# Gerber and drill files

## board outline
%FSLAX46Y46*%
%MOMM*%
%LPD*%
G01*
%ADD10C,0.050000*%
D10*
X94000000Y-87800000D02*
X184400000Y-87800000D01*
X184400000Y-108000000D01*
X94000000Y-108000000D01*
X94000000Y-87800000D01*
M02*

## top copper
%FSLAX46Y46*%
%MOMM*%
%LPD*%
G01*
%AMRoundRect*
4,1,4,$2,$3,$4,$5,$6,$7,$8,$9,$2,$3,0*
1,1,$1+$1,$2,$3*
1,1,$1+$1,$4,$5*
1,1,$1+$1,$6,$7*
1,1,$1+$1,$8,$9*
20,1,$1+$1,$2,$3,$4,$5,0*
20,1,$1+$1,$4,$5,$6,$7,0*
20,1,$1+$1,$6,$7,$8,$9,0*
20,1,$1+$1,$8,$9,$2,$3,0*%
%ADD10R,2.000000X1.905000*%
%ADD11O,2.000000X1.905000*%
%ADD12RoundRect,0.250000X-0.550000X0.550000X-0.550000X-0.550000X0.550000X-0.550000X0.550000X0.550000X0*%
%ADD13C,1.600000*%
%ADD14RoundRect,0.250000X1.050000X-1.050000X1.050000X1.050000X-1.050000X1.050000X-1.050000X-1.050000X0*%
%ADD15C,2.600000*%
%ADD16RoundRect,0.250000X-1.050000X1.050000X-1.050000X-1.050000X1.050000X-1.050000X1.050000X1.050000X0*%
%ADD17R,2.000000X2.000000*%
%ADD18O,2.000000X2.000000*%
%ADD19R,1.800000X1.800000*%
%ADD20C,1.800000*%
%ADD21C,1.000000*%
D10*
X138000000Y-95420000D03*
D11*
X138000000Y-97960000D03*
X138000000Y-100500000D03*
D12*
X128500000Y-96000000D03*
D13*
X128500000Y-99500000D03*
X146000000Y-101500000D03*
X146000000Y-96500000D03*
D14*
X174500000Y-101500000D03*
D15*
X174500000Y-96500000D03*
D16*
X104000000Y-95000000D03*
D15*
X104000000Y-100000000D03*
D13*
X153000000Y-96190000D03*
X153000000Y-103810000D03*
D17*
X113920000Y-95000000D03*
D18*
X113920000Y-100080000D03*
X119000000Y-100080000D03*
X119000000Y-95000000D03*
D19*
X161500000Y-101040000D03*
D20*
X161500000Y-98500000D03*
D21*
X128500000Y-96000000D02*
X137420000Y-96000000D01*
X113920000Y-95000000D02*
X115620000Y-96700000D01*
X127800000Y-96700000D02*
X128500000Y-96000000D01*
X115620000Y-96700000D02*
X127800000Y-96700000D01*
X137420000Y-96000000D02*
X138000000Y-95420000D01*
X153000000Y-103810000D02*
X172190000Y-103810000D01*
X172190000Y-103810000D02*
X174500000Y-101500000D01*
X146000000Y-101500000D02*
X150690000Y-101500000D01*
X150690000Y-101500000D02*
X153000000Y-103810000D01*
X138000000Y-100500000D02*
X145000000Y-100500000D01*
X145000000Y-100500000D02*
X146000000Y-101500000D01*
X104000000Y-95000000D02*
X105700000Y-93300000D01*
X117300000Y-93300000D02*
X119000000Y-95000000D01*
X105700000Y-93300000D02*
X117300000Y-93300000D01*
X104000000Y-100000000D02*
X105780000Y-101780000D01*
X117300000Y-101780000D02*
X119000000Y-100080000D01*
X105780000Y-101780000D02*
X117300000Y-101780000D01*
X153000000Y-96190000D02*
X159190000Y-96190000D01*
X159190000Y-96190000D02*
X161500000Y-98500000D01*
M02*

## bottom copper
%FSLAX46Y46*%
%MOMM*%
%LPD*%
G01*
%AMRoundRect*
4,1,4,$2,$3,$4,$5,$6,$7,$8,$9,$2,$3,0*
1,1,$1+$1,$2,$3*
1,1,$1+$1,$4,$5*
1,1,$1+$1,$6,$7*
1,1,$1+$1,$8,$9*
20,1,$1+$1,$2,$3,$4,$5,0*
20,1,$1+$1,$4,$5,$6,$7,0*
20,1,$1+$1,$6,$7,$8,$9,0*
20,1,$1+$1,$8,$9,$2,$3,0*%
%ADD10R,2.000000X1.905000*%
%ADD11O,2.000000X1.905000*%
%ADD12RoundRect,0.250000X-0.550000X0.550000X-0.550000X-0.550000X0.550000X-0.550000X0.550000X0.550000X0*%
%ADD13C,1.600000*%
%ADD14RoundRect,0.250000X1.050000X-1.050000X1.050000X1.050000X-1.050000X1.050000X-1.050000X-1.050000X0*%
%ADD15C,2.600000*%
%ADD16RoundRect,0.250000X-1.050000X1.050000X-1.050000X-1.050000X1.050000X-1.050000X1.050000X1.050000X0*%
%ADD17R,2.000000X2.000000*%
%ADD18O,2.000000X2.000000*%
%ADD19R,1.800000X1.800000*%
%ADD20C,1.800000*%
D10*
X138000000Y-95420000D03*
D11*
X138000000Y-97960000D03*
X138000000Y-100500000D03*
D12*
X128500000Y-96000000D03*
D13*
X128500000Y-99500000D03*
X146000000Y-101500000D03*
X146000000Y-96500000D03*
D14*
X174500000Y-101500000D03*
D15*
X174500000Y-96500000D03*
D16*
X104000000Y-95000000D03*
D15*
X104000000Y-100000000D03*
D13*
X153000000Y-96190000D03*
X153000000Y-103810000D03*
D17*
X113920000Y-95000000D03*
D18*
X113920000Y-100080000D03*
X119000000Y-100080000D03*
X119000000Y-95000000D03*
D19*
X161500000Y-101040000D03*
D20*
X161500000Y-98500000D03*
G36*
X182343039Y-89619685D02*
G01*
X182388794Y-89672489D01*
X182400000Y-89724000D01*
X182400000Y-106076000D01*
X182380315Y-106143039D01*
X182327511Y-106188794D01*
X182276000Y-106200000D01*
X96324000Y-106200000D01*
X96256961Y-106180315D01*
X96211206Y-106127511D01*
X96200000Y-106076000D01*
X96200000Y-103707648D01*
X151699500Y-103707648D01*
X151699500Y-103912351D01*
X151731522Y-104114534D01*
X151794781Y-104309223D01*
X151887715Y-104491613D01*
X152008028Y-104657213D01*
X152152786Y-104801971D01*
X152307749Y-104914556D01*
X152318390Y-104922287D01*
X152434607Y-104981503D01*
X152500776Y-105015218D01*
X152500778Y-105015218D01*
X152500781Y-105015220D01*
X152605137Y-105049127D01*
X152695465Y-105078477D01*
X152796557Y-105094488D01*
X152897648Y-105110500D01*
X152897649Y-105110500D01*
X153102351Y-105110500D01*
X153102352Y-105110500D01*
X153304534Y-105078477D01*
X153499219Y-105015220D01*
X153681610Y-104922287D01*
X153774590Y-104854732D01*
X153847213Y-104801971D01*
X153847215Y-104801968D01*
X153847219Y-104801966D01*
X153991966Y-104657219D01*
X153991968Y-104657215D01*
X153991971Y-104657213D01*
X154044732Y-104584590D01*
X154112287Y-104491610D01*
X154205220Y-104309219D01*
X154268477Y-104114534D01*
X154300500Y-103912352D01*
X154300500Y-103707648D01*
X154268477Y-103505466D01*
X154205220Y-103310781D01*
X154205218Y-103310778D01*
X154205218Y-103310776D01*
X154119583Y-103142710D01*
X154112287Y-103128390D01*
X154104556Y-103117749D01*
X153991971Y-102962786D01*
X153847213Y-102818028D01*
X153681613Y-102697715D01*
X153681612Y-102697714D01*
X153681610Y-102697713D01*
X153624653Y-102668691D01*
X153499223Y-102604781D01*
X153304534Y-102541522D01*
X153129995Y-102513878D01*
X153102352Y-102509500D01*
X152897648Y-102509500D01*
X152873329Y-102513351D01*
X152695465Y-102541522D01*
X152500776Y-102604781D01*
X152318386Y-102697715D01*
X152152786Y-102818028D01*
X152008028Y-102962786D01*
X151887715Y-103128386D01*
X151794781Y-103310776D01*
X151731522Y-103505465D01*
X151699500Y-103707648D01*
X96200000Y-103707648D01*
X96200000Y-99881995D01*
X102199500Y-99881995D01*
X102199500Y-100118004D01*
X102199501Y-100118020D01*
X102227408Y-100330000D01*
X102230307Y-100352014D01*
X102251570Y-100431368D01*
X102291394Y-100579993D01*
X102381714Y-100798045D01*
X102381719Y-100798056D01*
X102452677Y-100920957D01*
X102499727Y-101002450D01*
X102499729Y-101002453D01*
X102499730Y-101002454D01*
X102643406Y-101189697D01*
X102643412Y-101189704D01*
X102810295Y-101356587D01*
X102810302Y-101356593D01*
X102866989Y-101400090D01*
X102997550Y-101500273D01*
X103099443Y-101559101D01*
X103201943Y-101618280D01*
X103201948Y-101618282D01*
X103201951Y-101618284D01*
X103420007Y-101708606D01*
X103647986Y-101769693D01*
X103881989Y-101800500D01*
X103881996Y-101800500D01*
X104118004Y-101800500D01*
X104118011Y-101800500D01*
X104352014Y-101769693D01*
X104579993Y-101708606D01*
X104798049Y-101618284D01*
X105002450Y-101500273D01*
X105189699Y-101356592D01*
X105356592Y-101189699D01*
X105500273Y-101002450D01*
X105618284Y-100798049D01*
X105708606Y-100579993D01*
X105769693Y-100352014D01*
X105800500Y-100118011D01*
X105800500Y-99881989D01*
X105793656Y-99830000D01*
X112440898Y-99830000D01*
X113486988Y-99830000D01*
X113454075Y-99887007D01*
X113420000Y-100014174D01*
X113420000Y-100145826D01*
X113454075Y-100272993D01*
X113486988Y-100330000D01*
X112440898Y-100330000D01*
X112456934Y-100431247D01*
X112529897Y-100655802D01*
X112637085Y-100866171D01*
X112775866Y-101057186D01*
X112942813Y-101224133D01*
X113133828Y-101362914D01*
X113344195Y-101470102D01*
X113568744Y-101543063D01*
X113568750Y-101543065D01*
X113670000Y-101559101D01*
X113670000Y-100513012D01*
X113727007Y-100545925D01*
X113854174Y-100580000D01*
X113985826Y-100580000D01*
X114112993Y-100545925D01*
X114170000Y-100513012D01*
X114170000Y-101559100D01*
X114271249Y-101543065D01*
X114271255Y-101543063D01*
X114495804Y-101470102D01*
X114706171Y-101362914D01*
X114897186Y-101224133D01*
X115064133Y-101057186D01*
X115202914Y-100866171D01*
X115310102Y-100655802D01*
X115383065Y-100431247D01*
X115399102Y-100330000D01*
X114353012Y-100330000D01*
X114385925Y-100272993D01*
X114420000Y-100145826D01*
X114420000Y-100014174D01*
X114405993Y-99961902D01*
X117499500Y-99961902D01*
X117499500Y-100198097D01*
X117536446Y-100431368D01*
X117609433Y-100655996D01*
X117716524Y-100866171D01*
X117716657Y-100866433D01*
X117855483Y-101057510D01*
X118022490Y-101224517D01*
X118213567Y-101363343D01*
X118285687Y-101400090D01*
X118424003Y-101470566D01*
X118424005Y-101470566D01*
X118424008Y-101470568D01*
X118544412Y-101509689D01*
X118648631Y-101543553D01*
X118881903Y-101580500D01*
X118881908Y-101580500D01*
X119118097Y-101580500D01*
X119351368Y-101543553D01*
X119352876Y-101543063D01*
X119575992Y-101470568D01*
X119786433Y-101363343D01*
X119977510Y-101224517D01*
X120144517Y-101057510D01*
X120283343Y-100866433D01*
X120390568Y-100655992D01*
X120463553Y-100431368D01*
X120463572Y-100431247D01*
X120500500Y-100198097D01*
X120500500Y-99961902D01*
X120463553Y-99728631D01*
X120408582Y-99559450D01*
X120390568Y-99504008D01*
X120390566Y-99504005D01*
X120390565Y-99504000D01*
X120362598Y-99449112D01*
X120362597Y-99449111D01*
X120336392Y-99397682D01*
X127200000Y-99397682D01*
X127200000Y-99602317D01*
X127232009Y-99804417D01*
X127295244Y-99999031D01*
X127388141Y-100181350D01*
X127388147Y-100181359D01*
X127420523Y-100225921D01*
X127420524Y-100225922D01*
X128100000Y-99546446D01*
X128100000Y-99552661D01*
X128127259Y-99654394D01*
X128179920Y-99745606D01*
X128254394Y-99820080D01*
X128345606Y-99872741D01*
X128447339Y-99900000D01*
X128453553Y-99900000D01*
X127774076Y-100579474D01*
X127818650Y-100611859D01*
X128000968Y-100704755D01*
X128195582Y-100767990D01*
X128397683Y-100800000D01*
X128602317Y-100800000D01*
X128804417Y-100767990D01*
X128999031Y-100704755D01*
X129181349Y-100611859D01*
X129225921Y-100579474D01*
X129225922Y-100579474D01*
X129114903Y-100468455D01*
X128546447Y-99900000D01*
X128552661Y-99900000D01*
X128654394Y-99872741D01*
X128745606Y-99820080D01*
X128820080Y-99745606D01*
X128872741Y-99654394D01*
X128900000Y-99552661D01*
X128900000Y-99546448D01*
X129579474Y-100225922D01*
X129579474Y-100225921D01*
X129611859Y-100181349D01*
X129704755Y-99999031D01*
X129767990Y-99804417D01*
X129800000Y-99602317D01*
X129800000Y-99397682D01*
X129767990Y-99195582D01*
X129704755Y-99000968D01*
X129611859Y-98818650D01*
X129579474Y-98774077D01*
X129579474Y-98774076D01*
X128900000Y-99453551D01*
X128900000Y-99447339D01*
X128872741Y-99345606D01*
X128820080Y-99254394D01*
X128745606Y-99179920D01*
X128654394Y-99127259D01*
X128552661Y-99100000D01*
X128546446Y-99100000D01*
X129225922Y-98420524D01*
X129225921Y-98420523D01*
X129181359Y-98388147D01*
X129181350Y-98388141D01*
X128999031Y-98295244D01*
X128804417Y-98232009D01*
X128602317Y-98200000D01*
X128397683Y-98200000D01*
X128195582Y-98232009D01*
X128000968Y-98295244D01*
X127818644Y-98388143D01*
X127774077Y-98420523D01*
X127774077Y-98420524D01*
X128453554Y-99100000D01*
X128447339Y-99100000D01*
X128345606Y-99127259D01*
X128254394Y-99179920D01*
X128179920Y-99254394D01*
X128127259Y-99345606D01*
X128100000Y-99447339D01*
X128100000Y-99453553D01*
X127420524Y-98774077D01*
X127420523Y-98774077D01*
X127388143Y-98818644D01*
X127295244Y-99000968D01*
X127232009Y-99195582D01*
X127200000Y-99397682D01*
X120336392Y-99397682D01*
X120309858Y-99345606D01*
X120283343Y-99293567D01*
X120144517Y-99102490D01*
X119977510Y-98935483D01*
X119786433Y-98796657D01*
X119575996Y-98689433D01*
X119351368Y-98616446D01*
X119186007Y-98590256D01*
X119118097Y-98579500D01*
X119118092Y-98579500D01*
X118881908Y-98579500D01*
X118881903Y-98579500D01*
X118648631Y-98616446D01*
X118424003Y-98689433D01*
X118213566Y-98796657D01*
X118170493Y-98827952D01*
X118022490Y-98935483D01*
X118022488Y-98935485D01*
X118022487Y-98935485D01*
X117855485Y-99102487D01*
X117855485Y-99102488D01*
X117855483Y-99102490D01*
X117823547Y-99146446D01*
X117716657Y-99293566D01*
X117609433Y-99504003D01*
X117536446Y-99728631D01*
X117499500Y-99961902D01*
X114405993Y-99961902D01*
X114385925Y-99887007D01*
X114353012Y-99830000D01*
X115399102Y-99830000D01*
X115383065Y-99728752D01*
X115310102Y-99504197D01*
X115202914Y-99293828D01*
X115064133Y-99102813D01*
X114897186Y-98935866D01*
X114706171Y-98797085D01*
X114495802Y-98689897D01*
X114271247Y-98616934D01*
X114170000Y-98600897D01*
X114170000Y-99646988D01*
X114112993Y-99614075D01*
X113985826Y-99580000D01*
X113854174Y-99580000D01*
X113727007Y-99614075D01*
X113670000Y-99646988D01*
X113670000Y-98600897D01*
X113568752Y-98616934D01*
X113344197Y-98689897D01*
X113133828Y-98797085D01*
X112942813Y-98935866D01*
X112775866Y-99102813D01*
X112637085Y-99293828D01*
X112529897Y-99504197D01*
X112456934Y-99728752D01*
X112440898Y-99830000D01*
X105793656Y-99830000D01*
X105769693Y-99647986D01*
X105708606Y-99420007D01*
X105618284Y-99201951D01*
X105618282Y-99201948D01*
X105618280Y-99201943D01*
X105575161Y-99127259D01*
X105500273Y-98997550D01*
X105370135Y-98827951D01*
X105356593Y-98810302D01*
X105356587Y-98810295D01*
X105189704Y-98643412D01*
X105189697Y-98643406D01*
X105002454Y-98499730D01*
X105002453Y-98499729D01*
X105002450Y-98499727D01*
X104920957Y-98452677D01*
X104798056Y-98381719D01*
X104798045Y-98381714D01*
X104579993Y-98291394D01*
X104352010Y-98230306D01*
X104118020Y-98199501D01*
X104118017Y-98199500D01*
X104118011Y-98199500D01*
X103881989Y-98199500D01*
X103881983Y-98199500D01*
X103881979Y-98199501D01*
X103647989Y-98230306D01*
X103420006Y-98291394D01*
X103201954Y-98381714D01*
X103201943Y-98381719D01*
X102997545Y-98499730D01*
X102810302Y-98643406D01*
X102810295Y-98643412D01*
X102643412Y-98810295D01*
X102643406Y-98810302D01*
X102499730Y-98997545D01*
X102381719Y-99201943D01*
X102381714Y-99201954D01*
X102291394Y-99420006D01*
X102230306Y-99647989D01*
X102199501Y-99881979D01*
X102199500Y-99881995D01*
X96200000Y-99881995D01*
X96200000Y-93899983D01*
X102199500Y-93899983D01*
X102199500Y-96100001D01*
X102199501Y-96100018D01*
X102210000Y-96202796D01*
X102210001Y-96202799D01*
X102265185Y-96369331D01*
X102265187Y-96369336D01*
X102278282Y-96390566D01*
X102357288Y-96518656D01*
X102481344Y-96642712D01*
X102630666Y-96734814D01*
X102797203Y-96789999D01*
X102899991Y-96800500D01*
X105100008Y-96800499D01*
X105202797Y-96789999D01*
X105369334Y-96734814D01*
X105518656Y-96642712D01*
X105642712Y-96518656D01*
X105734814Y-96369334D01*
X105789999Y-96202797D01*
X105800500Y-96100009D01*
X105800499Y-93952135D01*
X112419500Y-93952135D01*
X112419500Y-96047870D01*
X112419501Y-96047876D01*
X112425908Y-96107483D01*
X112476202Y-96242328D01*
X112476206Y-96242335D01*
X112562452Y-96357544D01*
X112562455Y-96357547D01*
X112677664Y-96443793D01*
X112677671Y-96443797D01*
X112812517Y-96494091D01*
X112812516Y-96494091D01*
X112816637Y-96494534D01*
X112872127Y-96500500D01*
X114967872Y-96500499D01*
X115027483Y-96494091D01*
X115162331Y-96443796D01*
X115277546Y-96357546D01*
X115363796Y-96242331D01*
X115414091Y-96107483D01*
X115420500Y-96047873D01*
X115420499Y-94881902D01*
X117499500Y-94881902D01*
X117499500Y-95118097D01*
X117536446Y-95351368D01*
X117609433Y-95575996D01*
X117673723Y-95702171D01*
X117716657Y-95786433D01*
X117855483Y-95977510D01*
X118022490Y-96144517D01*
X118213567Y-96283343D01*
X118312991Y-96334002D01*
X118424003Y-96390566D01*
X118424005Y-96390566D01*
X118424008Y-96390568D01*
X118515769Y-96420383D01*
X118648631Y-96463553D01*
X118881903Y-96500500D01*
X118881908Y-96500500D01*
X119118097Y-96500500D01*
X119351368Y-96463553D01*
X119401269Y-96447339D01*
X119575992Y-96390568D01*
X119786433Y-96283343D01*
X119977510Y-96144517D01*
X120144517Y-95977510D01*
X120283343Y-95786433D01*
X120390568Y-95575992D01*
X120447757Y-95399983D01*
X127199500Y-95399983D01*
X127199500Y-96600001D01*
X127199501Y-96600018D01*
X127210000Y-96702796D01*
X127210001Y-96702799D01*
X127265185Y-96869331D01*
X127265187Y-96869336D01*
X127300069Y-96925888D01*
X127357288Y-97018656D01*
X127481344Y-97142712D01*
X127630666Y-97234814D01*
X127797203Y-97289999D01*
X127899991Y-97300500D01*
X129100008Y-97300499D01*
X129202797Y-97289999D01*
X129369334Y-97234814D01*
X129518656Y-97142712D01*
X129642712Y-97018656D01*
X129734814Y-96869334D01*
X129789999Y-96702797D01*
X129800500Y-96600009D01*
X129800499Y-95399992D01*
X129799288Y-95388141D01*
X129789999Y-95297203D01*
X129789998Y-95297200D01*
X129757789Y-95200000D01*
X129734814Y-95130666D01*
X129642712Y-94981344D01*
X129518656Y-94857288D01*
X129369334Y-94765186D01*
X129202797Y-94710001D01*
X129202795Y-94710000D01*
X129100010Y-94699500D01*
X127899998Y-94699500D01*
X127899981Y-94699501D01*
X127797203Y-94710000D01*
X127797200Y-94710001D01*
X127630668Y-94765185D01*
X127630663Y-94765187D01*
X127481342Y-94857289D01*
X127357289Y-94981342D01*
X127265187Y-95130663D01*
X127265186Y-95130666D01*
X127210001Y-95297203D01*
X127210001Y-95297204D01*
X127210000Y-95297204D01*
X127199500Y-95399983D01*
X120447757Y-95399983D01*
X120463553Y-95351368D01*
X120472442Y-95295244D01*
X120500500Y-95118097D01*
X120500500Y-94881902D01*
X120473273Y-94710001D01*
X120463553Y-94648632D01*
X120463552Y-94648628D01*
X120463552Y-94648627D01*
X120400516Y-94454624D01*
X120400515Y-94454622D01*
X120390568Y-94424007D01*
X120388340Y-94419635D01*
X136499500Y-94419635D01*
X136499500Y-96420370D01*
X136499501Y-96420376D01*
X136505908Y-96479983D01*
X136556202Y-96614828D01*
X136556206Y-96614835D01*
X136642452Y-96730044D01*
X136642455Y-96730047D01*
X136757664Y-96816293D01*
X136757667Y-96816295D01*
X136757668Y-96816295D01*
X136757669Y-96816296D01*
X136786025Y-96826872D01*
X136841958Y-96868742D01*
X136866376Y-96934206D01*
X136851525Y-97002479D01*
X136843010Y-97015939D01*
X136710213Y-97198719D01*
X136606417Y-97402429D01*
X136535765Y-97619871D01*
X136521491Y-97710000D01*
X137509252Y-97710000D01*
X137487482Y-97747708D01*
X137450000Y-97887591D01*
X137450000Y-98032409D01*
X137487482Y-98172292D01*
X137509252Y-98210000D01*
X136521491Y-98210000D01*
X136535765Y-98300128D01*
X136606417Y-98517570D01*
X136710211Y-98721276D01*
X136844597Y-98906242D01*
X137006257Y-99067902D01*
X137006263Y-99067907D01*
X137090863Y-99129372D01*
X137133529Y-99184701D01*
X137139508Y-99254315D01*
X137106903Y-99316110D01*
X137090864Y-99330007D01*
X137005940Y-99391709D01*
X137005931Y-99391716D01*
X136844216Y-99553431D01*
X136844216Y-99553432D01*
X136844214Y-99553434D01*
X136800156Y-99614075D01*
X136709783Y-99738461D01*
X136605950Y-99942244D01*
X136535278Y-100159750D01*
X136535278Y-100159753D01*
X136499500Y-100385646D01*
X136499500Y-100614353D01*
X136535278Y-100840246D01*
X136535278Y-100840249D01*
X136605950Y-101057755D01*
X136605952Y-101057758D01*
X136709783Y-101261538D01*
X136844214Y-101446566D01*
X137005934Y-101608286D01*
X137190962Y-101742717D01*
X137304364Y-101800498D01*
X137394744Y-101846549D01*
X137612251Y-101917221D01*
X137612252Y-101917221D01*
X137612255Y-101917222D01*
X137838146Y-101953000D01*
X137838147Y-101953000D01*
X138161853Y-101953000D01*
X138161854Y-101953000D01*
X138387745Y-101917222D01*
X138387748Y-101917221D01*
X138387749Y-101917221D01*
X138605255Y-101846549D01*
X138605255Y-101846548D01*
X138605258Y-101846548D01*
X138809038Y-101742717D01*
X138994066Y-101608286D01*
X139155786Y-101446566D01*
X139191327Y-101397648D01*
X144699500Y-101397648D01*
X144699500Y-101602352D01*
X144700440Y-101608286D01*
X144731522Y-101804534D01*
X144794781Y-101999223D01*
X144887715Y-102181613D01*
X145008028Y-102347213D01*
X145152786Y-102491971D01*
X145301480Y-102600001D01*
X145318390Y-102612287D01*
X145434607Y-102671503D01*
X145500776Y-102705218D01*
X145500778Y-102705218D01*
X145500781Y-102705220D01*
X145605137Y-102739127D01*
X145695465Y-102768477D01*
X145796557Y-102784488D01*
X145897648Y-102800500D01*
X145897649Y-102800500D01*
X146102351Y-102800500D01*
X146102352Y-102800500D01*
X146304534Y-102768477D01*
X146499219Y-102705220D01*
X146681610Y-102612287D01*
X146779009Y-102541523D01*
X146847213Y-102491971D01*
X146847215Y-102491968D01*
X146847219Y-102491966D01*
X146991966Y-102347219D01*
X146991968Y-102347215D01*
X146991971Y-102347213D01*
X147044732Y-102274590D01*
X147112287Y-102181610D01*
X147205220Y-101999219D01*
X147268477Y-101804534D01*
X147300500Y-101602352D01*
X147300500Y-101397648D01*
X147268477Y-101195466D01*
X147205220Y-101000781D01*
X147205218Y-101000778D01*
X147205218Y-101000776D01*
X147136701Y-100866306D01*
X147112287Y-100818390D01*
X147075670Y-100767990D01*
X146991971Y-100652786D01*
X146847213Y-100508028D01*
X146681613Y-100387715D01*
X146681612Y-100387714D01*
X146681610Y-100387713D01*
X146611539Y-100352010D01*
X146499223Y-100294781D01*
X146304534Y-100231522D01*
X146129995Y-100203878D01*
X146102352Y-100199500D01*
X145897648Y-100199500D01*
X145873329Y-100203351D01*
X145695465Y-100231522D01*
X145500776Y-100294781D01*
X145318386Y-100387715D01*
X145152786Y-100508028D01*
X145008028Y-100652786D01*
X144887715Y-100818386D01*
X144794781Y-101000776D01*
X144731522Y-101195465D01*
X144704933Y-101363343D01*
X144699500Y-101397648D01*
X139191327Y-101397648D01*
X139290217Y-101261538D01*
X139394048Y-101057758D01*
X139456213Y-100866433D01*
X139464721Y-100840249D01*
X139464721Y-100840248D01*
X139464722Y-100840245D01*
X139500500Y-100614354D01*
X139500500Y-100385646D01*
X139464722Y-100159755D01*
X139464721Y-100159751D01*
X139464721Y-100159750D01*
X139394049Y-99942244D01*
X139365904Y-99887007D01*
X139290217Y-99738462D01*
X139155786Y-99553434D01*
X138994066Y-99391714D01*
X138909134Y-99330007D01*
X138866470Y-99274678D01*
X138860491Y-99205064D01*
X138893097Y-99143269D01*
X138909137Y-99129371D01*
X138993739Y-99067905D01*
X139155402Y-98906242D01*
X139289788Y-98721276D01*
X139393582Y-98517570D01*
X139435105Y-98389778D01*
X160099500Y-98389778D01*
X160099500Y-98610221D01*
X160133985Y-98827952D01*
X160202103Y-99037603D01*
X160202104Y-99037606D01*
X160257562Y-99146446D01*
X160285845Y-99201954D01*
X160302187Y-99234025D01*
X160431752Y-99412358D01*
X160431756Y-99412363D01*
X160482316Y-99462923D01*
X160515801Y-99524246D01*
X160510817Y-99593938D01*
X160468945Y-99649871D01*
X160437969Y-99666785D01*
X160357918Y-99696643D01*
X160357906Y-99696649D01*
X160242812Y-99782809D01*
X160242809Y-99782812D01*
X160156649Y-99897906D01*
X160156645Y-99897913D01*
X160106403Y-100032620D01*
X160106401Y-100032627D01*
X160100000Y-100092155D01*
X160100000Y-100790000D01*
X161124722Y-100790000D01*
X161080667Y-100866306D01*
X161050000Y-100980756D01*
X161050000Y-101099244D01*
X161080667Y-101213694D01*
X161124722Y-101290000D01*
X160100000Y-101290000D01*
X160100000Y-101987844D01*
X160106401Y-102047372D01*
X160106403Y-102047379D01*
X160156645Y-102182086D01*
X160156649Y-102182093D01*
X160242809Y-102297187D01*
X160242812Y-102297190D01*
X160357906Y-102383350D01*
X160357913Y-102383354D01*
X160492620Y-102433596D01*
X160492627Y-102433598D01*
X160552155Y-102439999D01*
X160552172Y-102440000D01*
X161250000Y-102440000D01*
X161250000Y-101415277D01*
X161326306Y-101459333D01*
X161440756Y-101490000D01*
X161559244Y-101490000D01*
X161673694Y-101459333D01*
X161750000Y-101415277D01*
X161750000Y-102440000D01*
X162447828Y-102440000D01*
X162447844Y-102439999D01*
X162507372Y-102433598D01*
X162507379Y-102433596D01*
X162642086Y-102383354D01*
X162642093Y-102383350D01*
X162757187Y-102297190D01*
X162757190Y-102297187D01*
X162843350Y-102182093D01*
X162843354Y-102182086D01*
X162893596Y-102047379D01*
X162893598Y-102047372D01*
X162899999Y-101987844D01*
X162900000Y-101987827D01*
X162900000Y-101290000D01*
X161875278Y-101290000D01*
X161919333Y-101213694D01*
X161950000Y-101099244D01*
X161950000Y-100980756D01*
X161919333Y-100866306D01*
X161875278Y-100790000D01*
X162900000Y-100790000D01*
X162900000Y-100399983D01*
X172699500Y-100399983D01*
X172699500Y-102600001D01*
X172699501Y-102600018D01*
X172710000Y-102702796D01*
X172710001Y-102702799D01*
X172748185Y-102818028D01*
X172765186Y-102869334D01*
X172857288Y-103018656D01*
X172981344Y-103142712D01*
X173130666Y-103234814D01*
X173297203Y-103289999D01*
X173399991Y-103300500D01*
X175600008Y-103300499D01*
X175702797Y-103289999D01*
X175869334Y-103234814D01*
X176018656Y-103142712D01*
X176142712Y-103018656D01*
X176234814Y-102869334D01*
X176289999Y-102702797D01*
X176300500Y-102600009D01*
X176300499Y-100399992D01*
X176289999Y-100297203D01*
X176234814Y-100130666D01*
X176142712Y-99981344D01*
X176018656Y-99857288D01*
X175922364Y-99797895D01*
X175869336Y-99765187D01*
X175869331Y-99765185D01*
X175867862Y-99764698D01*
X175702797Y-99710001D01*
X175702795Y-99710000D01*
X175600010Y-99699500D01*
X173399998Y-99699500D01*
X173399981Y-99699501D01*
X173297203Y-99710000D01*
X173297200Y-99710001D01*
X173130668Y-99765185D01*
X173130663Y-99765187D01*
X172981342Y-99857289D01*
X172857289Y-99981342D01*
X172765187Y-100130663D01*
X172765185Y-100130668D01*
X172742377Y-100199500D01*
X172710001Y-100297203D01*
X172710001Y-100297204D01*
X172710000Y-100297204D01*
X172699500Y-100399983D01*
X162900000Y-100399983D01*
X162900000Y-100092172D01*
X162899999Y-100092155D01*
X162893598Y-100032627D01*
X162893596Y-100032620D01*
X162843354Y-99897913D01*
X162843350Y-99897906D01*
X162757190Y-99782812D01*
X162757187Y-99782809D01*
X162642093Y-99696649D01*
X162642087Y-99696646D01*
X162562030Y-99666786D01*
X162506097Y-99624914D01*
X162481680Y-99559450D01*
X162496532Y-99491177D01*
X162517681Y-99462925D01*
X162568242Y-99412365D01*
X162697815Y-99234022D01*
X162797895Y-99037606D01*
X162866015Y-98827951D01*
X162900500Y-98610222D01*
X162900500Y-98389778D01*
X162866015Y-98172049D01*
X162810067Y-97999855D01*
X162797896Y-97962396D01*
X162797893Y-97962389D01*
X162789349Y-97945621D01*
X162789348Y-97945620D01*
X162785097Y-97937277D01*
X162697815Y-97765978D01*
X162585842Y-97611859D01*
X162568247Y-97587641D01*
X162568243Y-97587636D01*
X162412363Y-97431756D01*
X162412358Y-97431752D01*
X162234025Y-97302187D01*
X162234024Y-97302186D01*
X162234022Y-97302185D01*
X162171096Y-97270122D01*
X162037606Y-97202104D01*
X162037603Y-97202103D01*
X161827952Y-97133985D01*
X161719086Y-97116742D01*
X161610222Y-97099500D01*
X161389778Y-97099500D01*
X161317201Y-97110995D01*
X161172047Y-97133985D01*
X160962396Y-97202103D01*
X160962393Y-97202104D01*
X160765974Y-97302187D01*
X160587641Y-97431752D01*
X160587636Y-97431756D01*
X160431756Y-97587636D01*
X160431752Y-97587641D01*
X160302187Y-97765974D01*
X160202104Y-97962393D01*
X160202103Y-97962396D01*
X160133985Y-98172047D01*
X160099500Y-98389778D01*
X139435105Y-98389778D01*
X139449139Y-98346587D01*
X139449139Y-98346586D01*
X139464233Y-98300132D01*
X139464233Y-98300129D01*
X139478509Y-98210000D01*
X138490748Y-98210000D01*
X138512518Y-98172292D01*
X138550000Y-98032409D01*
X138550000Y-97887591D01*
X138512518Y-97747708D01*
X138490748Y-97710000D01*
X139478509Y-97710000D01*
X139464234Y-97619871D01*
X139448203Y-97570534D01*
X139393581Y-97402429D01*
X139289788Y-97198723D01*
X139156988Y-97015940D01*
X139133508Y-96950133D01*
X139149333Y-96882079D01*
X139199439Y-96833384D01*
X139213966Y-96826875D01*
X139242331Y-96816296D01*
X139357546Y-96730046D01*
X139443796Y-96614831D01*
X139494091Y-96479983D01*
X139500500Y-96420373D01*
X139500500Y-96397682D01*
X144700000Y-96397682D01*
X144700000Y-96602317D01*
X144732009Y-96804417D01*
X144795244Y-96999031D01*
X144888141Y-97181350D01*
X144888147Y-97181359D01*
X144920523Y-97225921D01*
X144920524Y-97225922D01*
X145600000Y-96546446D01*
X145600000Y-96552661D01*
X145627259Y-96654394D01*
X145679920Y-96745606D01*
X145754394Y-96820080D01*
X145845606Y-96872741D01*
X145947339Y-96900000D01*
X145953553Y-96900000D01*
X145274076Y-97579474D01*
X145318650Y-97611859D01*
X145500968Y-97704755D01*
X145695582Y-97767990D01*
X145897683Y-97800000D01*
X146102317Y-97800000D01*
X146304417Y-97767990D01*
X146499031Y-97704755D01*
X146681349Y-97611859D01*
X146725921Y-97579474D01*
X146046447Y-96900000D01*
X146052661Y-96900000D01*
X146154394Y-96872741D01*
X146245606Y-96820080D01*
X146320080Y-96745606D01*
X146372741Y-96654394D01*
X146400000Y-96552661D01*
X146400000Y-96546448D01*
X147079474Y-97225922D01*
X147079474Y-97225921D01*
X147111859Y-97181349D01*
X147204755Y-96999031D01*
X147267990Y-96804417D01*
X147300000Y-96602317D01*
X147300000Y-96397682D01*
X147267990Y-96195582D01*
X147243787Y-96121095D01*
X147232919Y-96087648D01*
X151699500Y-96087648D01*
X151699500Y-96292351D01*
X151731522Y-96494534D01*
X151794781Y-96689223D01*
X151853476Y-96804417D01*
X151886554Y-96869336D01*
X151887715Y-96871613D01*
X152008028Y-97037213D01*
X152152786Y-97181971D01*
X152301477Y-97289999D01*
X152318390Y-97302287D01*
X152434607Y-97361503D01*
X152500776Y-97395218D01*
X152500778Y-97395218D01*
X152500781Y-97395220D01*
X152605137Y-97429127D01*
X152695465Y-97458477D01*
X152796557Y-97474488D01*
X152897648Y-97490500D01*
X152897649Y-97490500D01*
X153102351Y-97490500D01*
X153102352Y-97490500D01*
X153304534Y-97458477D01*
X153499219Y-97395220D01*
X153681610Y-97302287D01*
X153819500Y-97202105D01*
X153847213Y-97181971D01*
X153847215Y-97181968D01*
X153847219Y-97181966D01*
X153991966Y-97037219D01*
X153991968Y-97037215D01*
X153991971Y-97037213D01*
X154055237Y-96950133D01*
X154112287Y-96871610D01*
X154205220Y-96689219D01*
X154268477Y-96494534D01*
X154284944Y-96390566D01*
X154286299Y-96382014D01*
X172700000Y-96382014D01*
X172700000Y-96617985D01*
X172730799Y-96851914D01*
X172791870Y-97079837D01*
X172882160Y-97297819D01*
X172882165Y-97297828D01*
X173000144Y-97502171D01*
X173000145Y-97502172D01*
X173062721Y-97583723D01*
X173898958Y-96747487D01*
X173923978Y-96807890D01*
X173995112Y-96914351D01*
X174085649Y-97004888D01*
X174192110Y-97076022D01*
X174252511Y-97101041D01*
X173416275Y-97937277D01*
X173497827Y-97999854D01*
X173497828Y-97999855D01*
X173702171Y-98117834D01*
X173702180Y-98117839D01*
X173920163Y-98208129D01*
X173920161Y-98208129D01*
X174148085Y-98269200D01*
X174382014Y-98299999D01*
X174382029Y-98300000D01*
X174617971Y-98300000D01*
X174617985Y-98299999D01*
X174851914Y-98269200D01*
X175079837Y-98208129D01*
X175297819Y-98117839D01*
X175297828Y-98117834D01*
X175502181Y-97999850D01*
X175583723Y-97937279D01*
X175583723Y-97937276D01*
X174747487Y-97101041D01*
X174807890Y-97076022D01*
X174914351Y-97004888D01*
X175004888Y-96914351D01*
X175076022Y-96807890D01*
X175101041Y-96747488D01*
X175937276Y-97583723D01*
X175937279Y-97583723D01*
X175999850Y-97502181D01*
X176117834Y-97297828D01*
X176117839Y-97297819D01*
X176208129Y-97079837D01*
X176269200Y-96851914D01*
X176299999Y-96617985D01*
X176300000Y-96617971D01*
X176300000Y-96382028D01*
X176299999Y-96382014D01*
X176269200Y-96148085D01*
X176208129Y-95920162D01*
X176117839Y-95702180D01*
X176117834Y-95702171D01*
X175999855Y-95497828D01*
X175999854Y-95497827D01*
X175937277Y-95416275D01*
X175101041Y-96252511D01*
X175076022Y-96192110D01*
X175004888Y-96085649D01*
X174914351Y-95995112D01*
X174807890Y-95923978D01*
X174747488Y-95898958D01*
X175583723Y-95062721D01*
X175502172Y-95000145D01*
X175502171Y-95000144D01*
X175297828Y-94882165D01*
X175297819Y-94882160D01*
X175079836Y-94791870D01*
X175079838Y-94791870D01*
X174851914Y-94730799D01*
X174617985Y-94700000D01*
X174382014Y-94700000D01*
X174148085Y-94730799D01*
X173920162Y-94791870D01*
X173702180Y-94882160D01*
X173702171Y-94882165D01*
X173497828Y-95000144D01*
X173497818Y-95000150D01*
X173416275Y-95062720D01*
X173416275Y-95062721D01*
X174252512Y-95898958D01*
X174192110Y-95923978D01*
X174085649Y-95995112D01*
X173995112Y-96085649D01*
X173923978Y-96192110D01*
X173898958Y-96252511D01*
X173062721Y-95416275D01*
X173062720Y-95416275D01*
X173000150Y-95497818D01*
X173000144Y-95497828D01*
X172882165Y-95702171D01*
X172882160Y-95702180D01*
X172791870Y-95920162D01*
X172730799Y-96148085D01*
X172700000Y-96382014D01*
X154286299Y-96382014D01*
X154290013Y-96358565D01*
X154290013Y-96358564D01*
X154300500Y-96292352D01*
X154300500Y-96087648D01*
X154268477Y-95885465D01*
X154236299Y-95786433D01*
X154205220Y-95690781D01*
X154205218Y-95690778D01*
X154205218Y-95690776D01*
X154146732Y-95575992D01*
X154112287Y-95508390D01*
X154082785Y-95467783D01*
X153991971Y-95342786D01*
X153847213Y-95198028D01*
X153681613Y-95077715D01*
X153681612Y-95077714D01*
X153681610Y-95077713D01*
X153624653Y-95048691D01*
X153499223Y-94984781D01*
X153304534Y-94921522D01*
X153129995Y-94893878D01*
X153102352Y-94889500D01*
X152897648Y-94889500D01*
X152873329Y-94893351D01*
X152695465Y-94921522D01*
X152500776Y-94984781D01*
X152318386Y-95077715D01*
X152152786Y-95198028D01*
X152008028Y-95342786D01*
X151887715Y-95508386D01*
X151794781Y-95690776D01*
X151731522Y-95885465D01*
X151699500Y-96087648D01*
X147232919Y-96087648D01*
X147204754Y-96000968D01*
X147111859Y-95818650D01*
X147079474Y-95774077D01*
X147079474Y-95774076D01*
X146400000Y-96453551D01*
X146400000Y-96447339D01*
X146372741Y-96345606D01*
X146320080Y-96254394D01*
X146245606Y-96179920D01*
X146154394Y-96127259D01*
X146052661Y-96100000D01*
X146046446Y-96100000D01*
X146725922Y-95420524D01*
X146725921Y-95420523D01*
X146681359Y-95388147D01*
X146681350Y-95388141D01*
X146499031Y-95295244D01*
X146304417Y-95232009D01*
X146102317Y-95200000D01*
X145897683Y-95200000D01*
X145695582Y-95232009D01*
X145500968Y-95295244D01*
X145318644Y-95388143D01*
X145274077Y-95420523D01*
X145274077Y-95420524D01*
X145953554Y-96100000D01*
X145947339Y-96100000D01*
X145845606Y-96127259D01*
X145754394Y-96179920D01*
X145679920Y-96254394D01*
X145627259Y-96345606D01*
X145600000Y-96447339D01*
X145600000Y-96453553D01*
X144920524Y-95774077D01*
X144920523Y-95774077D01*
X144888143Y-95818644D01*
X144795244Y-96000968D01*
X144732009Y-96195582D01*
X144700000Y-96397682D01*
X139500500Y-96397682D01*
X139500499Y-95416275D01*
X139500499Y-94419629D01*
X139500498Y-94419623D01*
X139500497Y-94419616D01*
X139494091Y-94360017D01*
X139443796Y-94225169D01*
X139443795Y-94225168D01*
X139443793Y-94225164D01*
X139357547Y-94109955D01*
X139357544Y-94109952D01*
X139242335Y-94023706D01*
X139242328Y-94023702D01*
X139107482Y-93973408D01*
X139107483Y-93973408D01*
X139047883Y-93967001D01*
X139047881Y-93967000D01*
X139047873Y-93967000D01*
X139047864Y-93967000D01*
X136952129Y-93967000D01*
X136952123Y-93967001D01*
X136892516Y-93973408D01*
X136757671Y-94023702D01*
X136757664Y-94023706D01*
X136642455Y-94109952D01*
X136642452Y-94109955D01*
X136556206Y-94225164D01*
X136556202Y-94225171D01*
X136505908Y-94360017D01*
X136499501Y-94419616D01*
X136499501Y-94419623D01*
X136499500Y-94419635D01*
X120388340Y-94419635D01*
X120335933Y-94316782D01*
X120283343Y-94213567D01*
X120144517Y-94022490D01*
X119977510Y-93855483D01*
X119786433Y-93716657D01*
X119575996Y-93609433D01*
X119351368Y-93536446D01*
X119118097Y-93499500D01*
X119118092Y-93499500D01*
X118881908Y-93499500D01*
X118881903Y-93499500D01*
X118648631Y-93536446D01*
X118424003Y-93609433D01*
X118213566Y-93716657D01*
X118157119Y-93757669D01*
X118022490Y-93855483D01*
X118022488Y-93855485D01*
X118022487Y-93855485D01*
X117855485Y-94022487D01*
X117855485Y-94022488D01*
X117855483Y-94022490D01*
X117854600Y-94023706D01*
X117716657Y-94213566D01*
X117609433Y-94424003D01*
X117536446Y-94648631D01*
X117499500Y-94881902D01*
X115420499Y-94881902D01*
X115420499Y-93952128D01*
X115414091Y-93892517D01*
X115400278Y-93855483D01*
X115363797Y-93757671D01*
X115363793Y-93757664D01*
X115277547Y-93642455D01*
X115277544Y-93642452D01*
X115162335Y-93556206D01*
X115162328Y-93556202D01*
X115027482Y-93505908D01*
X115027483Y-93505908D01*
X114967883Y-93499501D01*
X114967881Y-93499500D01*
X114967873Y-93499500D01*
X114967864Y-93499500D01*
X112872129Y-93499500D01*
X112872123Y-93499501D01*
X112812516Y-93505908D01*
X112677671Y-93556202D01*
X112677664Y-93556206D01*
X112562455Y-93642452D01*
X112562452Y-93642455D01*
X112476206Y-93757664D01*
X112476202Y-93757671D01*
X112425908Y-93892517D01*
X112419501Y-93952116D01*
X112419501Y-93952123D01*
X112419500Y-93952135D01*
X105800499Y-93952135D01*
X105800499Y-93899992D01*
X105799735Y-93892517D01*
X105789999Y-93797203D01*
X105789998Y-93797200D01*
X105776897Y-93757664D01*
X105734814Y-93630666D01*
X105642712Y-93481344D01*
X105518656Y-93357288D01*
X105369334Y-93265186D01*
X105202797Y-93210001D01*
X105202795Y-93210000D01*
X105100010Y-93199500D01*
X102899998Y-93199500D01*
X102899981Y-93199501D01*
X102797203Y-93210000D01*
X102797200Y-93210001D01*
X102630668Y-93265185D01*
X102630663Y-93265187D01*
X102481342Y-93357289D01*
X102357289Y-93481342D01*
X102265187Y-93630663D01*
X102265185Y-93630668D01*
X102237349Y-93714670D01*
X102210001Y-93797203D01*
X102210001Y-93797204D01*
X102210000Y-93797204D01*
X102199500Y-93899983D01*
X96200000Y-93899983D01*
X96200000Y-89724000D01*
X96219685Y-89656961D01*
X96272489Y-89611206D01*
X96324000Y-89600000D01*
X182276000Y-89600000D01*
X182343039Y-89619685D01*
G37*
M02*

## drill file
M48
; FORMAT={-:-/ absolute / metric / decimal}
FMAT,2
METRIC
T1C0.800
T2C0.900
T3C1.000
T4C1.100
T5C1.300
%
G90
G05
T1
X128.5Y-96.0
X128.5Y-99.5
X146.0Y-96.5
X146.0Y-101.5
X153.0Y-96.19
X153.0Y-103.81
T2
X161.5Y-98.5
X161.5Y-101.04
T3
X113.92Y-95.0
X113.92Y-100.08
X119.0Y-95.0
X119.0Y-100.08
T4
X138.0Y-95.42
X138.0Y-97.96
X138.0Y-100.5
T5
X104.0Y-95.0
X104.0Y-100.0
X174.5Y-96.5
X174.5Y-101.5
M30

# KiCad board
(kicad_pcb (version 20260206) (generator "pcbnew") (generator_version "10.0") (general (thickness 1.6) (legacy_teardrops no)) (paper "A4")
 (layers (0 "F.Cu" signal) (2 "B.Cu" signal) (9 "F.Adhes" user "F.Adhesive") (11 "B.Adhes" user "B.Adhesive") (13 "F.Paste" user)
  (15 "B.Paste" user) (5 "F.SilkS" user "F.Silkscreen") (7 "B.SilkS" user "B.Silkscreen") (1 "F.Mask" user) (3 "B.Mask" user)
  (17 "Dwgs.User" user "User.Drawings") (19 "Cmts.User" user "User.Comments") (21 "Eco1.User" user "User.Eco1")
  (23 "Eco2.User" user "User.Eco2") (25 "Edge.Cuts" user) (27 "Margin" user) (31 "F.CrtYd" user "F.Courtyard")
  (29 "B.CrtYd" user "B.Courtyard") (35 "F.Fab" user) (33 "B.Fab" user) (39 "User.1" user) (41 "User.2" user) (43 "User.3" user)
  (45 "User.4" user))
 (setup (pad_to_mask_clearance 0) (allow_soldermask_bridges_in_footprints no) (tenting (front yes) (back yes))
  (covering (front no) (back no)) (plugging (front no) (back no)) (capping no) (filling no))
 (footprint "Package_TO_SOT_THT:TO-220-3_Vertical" (layer "F.Cu") (at 138 95.42 -90)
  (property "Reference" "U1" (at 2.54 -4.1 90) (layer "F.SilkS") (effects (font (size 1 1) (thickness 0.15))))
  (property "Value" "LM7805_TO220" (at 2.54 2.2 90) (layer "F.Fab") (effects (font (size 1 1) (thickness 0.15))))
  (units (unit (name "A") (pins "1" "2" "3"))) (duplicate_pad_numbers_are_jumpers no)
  (pad "1" thru_hole rect (at 0 0 270) (size 1.905 2) (drill 1.1) (layers "*.Cu" "*.Mask") (remove_unused_layers no) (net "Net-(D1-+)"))
  (pad "2" thru_hole oval (at 2.54 0 270) (size 1.905 2) (drill 1.1) (layers "*.Cu" "*.Mask") (remove_unused_layers no) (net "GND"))
  (pad "3" thru_hole oval (at 5.08 0 270) (size 1.905 2) (drill 1.1) (layers "*.Cu" "*.Mask") (remove_unused_layers no)
   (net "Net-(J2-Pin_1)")))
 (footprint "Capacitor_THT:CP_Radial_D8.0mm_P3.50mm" (layer "F.Cu") (at 128.5 96 -90)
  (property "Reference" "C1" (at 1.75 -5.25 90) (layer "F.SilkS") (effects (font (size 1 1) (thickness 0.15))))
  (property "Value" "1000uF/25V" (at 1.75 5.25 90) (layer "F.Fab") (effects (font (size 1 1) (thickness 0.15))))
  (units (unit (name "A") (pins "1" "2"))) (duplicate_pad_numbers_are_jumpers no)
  (pad "1" thru_hole roundrect (at 0 0 270) (size 1.6 1.6) (drill 0.8) (layers "*.Cu" "*.Mask") (remove_unused_layers no)
   (roundrect_rratio 0.15625) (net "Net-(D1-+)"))
  (pad "2" thru_hole circle (at 3.5 0 270) (size 1.6 1.6) (drill 0.8) (layers "*.Cu" "*.Mask") (remove_unused_layers no) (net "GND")))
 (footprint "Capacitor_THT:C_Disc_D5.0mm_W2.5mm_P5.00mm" (layer "F.Cu") (at 146 101.5 90)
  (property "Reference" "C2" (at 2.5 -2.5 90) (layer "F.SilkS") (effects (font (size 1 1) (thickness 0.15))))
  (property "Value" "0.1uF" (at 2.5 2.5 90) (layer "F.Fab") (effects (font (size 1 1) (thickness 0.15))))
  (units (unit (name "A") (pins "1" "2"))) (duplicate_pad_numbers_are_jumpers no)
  (pad "1" thru_hole circle (at 0 0 90) (size 1.6 1.6) (drill 0.8) (layers "*.Cu" "*.Mask") (remove_unused_layers no) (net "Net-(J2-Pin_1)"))
  (pad "2" thru_hole circle (at 5 0 90) (size 1.6 1.6) (drill 0.8) (layers "*.Cu" "*.Mask") (remove_unused_layers no) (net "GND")))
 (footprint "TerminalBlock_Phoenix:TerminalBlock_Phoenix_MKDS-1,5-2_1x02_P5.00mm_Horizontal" (layer "F.Cu") (at 174.5 101.5 90)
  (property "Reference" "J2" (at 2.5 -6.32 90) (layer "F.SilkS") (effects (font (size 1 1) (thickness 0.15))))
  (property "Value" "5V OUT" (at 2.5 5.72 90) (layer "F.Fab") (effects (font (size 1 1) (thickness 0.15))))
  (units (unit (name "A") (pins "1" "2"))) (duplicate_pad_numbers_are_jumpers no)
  (pad "1" thru_hole roundrect (at 0 0 90) (size 2.6 2.6) (drill 1.3) (layers "*.Cu" "*.Mask") (remove_unused_layers no)
   (roundrect_rratio 0.096154) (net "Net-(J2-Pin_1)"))
  (pad "2" thru_hole circle (at 5 0 90) (size 2.6 2.6) (drill 1.3) (layers "*.Cu" "*.Mask") (remove_unused_layers no) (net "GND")))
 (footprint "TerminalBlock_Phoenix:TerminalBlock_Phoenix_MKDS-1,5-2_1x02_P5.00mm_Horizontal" (layer "F.Cu") (at 104 95 -90)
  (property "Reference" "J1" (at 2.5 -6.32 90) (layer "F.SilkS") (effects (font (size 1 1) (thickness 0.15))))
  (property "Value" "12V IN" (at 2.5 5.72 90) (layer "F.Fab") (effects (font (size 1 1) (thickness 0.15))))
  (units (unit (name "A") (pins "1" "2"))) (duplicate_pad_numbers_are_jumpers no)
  (pad "1" thru_hole roundrect (at 0 0 270) (size 2.6 2.6) (drill 1.3) (layers "*.Cu" "*.Mask") (remove_unused_layers no)
   (roundrect_rratio 0.096154) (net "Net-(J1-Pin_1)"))
  (pad "2" thru_hole circle (at 5 0 270) (size 2.6 2.6) (drill 1.3) (layers "*.Cu" "*.Mask") (remove_unused_layers no)
   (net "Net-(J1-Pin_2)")))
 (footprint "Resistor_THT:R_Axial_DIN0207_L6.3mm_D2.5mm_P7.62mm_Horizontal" (layer "F.Cu") (at 153 96.19 -90)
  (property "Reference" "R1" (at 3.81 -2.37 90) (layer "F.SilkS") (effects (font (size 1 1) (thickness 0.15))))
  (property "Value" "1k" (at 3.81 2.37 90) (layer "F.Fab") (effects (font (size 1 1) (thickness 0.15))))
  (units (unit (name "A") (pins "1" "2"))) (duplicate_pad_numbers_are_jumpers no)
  (pad "1" thru_hole circle (at 0 0 270) (size 1.6 1.6) (drill 0.8) (layers "*.Cu" "*.Mask") (remove_unused_layers no) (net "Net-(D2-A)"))
  (pad "2" thru_hole circle (at 7.62 0 270) (size 1.6 1.6) (drill 0.8) (layers "*.Cu" "*.Mask") (remove_unused_layers no)
   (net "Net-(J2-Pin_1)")))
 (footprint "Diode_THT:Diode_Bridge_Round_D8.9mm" (layer "F.Cu") (at 113.92 95)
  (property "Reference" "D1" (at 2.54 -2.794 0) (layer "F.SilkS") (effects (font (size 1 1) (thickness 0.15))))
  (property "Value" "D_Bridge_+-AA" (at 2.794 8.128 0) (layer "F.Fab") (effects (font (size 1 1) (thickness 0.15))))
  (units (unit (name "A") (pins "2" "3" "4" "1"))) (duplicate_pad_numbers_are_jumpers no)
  (pad "1" thru_hole rect (at 0 0) (size 2 2) (drill 1) (layers "*.Cu" "*.Mask") (remove_unused_layers no) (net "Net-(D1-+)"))
  (pad "2" thru_hole oval (at 0 5.08) (size 2 2) (drill 1) (layers "*.Cu" "*.Mask") (remove_unused_layers no) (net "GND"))
  (pad "3" thru_hole oval (at 5.08 5.08) (size 2 2) (drill 1) (layers "*.Cu" "*.Mask") (remove_unused_layers no) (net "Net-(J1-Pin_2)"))
  (pad "4" thru_hole oval (at 5.08 0) (size 2 2) (drill 1) (layers "*.Cu" "*.Mask") (remove_unused_layers no) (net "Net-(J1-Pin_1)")))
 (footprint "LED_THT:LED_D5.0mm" (layer "F.Cu") (at 161.5 101.04 90)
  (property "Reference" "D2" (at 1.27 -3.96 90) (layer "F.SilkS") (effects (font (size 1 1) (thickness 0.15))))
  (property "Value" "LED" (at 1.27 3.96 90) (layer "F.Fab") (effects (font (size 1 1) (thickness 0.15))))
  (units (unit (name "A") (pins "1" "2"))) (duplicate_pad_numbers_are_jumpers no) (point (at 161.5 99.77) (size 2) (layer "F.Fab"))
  (pad "1" thru_hole rect (at 0 0 90) (size 1.8 1.8) (drill 0.9) (layers "*.Cu" "*.Mask") (remove_unused_layers no) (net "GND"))
  (pad "2" thru_hole circle (at 2.54 0 90) (size 1.8 1.8) (drill 0.9) (layers "*.Cu" "*.Mask") (remove_unused_layers no) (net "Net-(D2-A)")))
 (gr_rect (start 94 87.8) (end 184.4 108) (stroke (width 0.05) (type default)) (fill no) (layer "Edge.Cuts"))
 (segment (start 128.5 96) (end 137.42 96) (width 1) (layer "F.Cu") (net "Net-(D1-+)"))
 (segment (start 113.92 95) (end 115.62 96.7) (width 1) (layer "F.Cu") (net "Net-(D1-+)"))
 (segment (start 127.8 96.7) (end 128.5 96) (width 1) (layer "F.Cu") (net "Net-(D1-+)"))
 (segment (start 115.62 96.7) (end 127.8 96.7) (width 1) (layer "F.Cu") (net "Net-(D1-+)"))
 (segment (start 137.42 96) (end 138 95.42) (width 1) (layer "F.Cu") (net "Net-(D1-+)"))
 (segment (start 153 103.81) (end 172.19 103.81) (width 1) (layer "F.Cu") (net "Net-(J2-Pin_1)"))
 (segment (start 172.19 103.81) (end 174.5 101.5) (width 1) (layer "F.Cu") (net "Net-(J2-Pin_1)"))
 (segment (start 146 101.5) (end 150.69 101.5) (width 1) (layer "F.Cu") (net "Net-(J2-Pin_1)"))
 (segment (start 150.69 101.5) (end 153 103.81) (width 1) (layer "F.Cu") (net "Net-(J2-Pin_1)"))
 (segment (start 138 100.5) (end 145 100.5) (width 1) (layer "F.Cu") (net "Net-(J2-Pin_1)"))
 (segment (start 145 100.5) (end 146 101.5) (width 1) (layer "F.Cu") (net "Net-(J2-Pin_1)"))
 (segment (start 104 95) (end 105.7 93.3) (width 1) (layer "F.Cu") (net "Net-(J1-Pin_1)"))
 (segment (start 117.3 93.3) (end 119 95) (width 1) (layer "F.Cu") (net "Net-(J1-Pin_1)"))
 (segment (start 105.7 93.3) (end 117.3 93.3) (width 1) (layer "F.Cu") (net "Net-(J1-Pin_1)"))
 (segment (start 104 100) (end 105.78 101.78) (width 1) (layer "F.Cu") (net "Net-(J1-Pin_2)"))
 (segment (start 117.3 101.78) (end 119 100.08) (width 1) (layer "F.Cu") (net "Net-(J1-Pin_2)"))
 (segment (start 105.78 101.78) (end 117.3 101.78) (width 1) (layer "F.Cu") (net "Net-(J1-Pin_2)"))
 (segment (start 153 96.19) (end 159.19 96.19) (width 1) (layer "F.Cu") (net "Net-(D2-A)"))
 (segment (start 159.19 96.19) (end 161.5 98.5) (width 1) (layer "F.Cu") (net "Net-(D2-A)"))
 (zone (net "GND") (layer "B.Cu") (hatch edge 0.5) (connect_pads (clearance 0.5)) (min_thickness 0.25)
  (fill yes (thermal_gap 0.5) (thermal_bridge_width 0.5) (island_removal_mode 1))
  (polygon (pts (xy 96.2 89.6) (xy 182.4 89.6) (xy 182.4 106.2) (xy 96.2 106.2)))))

